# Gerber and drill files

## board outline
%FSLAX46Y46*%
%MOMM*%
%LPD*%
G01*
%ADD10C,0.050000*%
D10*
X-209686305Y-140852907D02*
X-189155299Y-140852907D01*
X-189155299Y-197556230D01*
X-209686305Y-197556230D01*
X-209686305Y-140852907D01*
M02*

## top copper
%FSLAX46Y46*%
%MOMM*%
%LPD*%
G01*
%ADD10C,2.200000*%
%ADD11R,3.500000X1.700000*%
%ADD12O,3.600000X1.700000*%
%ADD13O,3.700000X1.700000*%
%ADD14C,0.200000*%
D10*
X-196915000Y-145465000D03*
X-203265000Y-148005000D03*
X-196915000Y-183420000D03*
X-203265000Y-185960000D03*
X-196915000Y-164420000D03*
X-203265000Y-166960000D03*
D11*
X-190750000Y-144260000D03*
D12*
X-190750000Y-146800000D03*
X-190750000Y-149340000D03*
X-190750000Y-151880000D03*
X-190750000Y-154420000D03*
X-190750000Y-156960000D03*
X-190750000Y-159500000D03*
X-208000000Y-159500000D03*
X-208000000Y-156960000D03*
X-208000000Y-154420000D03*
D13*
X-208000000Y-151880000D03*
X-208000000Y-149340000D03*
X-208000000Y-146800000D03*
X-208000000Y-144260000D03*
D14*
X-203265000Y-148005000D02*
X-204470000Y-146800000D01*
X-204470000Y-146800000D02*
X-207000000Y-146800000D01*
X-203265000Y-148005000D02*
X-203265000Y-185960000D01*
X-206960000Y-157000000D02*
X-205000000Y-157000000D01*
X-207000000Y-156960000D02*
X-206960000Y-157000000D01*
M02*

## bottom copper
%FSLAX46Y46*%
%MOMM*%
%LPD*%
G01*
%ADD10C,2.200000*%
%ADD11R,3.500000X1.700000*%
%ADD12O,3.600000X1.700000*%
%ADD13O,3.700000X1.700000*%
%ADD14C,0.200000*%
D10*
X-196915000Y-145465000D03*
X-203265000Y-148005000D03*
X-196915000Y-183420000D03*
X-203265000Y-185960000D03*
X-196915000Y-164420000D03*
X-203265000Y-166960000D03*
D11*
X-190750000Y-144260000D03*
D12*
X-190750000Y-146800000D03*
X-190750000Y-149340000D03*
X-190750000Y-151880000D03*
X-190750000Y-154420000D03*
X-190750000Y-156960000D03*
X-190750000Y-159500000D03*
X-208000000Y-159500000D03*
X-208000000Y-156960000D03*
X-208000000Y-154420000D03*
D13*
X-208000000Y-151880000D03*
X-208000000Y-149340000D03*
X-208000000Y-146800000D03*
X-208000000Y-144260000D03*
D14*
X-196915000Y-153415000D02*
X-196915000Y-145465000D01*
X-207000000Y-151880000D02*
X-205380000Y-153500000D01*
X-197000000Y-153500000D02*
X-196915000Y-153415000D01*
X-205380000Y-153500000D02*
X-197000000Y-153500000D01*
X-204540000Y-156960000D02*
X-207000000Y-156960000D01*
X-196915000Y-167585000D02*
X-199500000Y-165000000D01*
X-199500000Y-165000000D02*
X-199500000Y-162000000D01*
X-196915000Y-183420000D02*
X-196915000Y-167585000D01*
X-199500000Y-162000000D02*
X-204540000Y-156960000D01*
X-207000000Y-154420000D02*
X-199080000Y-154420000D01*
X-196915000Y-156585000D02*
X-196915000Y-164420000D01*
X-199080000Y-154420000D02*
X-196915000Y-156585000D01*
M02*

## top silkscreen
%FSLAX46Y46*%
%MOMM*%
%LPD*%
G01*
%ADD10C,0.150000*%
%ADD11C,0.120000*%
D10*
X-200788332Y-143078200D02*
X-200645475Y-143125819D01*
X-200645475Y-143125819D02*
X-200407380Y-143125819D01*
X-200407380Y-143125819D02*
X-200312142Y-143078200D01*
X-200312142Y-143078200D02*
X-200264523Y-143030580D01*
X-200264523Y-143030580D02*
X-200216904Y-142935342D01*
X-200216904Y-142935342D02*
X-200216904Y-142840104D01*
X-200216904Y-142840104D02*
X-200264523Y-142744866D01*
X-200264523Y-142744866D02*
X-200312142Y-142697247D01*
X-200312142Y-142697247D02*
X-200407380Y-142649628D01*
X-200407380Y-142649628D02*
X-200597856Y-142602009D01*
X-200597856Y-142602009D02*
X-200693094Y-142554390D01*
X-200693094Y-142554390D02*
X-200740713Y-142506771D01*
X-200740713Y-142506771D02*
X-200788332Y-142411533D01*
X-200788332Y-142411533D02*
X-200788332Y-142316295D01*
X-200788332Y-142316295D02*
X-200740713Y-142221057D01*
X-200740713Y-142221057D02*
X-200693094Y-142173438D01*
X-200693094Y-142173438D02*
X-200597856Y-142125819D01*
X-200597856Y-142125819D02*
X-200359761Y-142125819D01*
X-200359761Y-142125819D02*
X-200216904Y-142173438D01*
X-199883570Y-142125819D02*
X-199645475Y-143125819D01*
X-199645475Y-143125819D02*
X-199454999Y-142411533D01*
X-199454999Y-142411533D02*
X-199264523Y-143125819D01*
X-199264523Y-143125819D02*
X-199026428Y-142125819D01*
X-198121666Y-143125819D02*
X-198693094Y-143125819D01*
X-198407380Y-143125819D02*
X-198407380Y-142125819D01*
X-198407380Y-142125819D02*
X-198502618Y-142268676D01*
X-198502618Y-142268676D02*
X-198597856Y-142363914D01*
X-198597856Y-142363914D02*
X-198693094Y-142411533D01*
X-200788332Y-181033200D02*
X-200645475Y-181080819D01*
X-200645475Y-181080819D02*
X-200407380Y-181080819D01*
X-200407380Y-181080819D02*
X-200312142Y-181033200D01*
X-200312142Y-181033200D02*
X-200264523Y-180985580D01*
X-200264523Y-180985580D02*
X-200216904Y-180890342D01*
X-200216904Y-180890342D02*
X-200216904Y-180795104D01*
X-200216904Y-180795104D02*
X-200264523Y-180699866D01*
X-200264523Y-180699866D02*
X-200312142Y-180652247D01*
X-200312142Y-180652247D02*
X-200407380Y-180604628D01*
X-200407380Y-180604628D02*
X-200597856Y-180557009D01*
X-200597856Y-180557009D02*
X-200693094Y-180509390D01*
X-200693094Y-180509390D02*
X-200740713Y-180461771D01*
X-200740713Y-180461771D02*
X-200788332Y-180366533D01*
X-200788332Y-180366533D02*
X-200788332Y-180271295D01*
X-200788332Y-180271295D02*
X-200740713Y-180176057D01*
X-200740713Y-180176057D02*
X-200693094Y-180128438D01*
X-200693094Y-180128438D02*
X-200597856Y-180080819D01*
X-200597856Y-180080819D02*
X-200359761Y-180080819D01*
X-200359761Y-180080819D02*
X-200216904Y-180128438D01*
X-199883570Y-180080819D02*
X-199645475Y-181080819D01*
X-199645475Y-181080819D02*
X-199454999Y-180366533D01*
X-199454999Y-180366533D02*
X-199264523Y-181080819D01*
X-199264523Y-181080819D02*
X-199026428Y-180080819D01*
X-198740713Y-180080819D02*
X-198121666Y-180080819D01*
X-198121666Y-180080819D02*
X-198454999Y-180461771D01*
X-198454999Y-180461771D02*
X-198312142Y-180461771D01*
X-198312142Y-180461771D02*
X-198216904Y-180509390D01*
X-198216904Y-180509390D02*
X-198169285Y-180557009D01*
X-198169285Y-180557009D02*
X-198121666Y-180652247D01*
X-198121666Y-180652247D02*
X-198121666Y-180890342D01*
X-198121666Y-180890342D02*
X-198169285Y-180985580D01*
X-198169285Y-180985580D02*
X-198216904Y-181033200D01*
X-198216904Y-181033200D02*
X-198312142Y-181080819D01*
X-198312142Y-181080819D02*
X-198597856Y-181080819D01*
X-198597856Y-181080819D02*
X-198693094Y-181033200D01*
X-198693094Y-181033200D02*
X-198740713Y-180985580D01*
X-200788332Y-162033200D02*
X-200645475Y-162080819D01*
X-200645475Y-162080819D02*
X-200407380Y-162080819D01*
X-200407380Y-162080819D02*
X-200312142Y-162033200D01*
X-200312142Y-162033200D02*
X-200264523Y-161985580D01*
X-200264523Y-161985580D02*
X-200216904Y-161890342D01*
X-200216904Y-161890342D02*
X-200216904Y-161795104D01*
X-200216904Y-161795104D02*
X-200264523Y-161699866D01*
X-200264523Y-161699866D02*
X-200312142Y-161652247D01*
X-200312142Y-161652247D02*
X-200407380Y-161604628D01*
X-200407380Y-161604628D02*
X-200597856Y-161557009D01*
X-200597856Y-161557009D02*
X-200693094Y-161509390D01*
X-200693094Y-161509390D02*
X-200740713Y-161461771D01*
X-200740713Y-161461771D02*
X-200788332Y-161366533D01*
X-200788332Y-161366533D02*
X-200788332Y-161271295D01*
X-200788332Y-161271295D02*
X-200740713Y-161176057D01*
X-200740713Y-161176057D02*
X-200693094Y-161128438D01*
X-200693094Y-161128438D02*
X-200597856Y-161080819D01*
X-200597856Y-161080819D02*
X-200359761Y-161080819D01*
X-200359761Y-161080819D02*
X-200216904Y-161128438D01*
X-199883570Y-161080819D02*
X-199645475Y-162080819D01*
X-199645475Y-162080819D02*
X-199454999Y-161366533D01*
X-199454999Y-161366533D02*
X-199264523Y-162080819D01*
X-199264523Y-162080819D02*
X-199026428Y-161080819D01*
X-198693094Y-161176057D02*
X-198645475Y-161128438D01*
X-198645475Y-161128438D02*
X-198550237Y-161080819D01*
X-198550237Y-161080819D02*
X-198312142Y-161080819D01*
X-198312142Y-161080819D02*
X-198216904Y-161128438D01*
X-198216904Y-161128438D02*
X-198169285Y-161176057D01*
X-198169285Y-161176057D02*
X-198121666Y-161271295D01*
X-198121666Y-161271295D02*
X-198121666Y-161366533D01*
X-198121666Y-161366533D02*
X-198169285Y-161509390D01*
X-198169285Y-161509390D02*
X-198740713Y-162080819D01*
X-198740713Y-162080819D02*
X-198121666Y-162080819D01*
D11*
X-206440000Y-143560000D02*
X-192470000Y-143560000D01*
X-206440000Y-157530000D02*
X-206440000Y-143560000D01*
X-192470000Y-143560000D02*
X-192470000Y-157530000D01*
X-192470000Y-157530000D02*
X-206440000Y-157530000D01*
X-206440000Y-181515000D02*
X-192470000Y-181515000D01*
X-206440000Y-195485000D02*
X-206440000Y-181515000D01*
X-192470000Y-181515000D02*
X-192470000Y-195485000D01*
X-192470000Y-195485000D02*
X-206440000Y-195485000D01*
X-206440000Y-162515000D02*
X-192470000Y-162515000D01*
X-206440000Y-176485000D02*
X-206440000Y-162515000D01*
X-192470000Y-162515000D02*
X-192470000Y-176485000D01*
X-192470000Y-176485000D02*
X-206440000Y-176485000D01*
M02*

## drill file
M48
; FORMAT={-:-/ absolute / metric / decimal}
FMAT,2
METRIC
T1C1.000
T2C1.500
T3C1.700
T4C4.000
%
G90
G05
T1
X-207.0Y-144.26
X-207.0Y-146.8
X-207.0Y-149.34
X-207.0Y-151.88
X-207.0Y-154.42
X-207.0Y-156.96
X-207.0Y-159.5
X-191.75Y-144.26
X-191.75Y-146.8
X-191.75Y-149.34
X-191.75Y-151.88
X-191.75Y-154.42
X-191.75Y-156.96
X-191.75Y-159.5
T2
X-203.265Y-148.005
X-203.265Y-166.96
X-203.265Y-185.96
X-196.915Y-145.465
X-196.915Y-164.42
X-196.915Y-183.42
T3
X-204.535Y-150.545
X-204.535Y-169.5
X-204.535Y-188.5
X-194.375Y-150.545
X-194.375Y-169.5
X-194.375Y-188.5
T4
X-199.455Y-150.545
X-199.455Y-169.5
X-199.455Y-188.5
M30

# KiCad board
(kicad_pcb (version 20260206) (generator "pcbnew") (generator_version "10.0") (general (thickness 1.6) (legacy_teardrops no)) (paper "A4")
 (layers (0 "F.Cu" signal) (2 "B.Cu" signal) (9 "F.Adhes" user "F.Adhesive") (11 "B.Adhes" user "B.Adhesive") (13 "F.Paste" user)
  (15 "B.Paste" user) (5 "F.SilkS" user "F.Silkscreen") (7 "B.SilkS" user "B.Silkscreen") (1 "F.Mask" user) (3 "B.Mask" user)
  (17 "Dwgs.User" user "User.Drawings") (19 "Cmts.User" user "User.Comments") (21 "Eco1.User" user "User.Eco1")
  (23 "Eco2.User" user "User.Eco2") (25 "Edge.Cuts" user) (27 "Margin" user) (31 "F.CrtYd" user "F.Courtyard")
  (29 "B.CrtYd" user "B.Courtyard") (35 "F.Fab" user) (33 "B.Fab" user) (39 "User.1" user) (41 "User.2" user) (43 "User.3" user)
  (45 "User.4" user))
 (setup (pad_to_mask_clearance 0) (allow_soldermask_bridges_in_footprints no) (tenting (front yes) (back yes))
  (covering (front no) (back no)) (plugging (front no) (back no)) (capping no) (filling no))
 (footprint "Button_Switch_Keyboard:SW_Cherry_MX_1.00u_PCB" (layer "F.Cu") (at -196.915 145.465)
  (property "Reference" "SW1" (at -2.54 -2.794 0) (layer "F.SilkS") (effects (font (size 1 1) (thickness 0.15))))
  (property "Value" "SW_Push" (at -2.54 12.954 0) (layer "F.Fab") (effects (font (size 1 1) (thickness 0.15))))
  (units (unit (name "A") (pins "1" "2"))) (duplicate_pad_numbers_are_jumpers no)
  (fp_line (start -9.525 -1.905) (end 4.445 -1.905) (stroke (width 0.12) (type solid)) (layer "F.SilkS"))
  (fp_line (start -9.525 12.065) (end -9.525 -1.905) (stroke (width 0.12) (type solid)) (layer "F.SilkS"))
  (fp_line (start 4.445 -1.905) (end 4.445 12.065) (stroke (width 0.12) (type solid)) (layer "F.SilkS"))
  (fp_line (start 4.445 12.065) (end -9.525 12.065) (stroke (width 0.12) (type solid)) (layer "F.SilkS"))
  (pad "" np_thru_hole circle (at -7.62 5.08) (size 1.7 1.7) (drill 1.7) (layers "*.Cu" "*.Mask"))
  (pad "" np_thru_hole circle (at -2.54 5.08) (size 4 4) (drill 4) (layers "*.Cu" "*.Mask"))
  (pad "" np_thru_hole circle (at 2.54 5.08) (size 1.7 1.7) (drill 1.7) (layers "*.Cu" "*.Mask"))
  (pad "1" thru_hole circle (at 0 0) (size 2.2 2.2) (drill 1.5) (layers "*.Cu" "*.Mask") (remove_unused_layers no)
   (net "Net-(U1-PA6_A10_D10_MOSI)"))
  (pad "2" thru_hole circle (at -6.35 2.54) (size 2.2 2.2) (drill 1.5) (layers "*.Cu" "*.Mask") (remove_unused_layers no) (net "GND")))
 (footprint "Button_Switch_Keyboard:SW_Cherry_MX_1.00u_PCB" (layer "F.Cu") (at -196.915 183.42)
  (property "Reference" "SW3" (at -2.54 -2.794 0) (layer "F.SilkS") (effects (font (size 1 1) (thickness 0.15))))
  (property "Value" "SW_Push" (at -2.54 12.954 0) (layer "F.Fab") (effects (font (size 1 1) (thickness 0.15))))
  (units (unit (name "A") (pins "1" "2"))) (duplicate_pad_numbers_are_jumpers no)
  (fp_line (start -9.525 -1.905) (end 4.445 -1.905) (stroke (width 0.12) (type solid)) (layer "F.SilkS"))
  (fp_line (start -9.525 12.065) (end -9.525 -1.905) (stroke (width 0.12) (type solid)) (layer "F.SilkS"))
  (fp_line (start 4.445 -1.905) (end 4.445 12.065) (stroke (width 0.12) (type solid)) (layer "F.SilkS"))
  (fp_line (start 4.445 12.065) (end -9.525 12.065) (stroke (width 0.12) (type solid)) (layer "F.SilkS"))
  (pad "" np_thru_hole circle (at -7.62 5.08) (size 1.7 1.7) (drill 1.7) (layers "*.Cu" "*.Mask"))
  (pad "" np_thru_hole circle (at -2.54 5.08) (size 4 4) (drill 4) (layers "*.Cu" "*.Mask"))
  (pad "" np_thru_hole circle (at 2.54 5.08) (size 1.7 1.7) (drill 1.7) (layers "*.Cu" "*.Mask"))
  (pad "1" thru_hole circle (at 0 0) (size 2.2 2.2) (drill 1.5) (layers "*.Cu" "*.Mask") (remove_unused_layers no)
   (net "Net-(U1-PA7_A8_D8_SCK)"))
  (pad "2" thru_hole circle (at -6.35 2.54) (size 2.2 2.2) (drill 1.5) (layers "*.Cu" "*.Mask") (remove_unused_layers no) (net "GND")))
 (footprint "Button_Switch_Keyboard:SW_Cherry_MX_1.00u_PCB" (layer "F.Cu") (at -196.915 164.42)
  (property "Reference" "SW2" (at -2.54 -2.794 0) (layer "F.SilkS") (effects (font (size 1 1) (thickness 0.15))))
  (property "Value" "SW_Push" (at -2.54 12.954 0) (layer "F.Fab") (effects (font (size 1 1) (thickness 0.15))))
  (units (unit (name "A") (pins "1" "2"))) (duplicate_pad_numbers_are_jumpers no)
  (fp_line (start -9.525 -1.905) (end 4.445 -1.905) (stroke (width 0.12) (type solid)) (layer "F.SilkS"))
  (fp_line (start -9.525 12.065) (end -9.525 -1.905) (stroke (width 0.12) (type solid)) (layer "F.SilkS"))
  (fp_line (start 4.445 -1.905) (end 4.445 12.065) (stroke (width 0.12) (type solid)) (layer "F.SilkS"))
  (fp_line (start 4.445 12.065) (end -9.525 12.065) (stroke (width 0.12) (type solid)) (layer "F.SilkS"))
  (pad "" np_thru_hole circle (at -7.62 5.08) (size 1.7 1.7) (drill 1.7) (layers "*.Cu" "*.Mask"))
  (pad "" np_thru_hole circle (at -2.54 5.08) (size 4 4) (drill 4) (layers "*.Cu" "*.Mask"))
  (pad "" np_thru_hole circle (at 2.54 5.08) (size 1.7 1.7) (drill 1.7) (layers "*.Cu" "*.Mask"))
  (pad "1" thru_hole circle (at 0 0) (size 2.2 2.2) (drill 1.5) (layers "*.Cu" "*.Mask") (remove_unused_layers no)
   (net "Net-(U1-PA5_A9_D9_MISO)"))
  (pad "2" thru_hole circle (at -6.35 2.54) (size 2.2 2.2) (drill 1.5) (layers "*.Cu" "*.Mask") (remove_unused_layers no) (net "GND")))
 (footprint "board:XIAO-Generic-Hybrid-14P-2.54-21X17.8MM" (layer "B.Cu") (at -199.375 151.88 180)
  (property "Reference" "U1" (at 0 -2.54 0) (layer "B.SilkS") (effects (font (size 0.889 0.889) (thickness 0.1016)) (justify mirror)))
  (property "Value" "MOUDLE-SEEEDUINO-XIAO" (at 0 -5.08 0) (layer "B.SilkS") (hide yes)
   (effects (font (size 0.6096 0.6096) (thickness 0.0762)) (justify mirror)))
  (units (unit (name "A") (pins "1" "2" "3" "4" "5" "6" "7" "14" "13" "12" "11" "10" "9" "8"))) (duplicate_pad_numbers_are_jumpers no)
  (pad "1" thru_hole rect (at -7.625 7.62 180) (size 3.5 1.7) (drill 1 (offset -1 0)) (layers "*.Cu" "*.Mask") (remove_unused_layers no)
   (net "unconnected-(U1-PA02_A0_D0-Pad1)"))
  (pad "2" thru_hole oval (at -7.625 5.08 180) (size 3.6 1.7) (drill 1 (offset -1 0)) (layers "*.Cu" "*.Mask") (remove_unused_layers no)
   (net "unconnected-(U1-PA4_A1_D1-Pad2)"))
  (pad "3" thru_hole oval (at -7.625 2.54 180) (size 3.6 1.7) (drill 1 (offset -1 0)) (layers "*.Cu" "*.Mask") (remove_unused_layers no)
   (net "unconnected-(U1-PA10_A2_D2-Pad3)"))
  (pad "4" thru_hole oval (at -7.625 0 180) (size 3.6 1.7) (drill 1 (offset -1 0)) (layers "*.Cu" "*.Mask") (remove_unused_layers no)
   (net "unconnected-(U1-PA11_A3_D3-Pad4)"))
  (pad "5" thru_hole oval (at -7.625 -2.54 180) (size 3.6 1.7) (drill 1 (offset -1 0)) (layers "*.Cu" "*.Mask") (remove_unused_layers no)
   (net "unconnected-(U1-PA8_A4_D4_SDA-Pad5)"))
  (pad "6" thru_hole oval (at -7.625 -5.08) (size 3.6 1.7) (drill 1 (offset 1 0)) (layers "*.Cu" "*.Mask") (remove_unused_layers no)
   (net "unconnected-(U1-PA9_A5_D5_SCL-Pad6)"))
  (pad "7" thru_hole oval (at -7.625 -7.62 180) (size 3.6 1.7) (drill 1 (offset -1 0)) (layers "*.Cu" "*.Mask") (remove_unused_layers no)
   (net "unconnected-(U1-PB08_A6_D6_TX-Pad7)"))
  (pad "8" thru_hole oval (at 7.625 -7.62 180) (size 3.6 1.7) (drill 1 (offset 1 0)) (layers "*.Cu" "*.Mask") (remove_unused_layers no)
   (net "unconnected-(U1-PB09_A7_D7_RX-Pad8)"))
  (pad "9" thru_hole oval (at 7.625 -5.08 180) (size 3.6 1.7) (drill 1 (offset 1 0)) (layers "*.Cu" "*.Mask") (remove_unused_layers no)
   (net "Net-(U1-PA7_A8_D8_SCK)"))
  (pad "10" thru_hole oval (at 7.625 -2.54 180) (size 3.6 1.7) (drill 1 (offset 1 0)) (layers "*.Cu" "*.Mask") (remove_unused_layers no)
   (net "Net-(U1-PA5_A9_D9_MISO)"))
  (pad "11" thru_hole oval (at 7.625 0 180) (size 3.7 1.7) (drill 1 (offset 1 0)) (layers "*.Cu" "*.Mask") (remove_unused_layers no)
   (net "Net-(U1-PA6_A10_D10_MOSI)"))
  (pad "12" thru_hole oval (at 7.625 2.54 180) (size 3.7 1.7) (drill 1 (offset 1 0)) (layers "*.Cu" "*.Mask") (remove_unused_layers no)
   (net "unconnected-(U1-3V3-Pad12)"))
  (pad "13" thru_hole oval (at 7.625 5.08 180) (size 3.7 1.7) (drill 1 (offset 1 0)) (layers "*.Cu" "*.Mask") (remove_unused_layers no)
   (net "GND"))
  (pad "14" thru_hole oval (at 7.625 7.62 180) (size 3.7 1.7) (drill 1 (offset 1 0)) (layers "*.Cu" "*.Mask") (remove_unused_layers no)
   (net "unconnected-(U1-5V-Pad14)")))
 (gr_rect (start -209.686305 140.852907) (end -189.155299 197.55623) (stroke (width 0.05) (type default)) (fill no) (layer "Edge.Cuts"))
 (segment (start -196.915 153.415) (end -196.915 145.465) (width 0.2) (layer "B.Cu") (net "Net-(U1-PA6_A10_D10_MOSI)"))
 (segment (start -207 151.88) (end -205.38 153.5) (width 0.2) (layer "B.Cu") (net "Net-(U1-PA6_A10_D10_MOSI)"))
 (segment (start -197 153.5) (end -196.915 153.415) (width 0.2) (layer "B.Cu") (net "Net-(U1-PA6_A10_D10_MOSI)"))
 (segment (start -205.38 153.5) (end -197 153.5) (width 0.2) (layer "B.Cu") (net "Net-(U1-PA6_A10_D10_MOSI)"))
 (segment (start -203.265 148.005) (end -204.47 146.8) (width 0.2) (layer "F.Cu") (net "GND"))
 (segment (start -204.47 146.8) (end -207 146.8) (width 0.2) (layer "F.Cu") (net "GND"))
 (segment (start -203.265 148.005) (end -203.265 185.96) (width 0.2) (layer "F.Cu") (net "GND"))
 (segment (start -206.96 157) (end -205 157) (width 0.2) (layer "F.Cu") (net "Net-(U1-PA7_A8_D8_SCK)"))
 (segment (start -207 156.96) (end -206.96 157) (width 0.2) (layer "F.Cu") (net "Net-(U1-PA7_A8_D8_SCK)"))
 (segment (start -204.54 156.96) (end -207 156.96) (width 0.2) (layer "B.Cu") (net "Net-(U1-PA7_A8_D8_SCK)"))
 (segment (start -196.915 167.585) (end -199.5 165) (width 0.2) (layer "B.Cu") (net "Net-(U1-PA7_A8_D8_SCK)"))
 (segment (start -199.5 165) (end -199.5 162) (width 0.2) (layer "B.Cu") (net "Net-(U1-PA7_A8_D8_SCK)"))
 (segment (start -196.915 183.42) (end -196.915 167.585) (width 0.2) (layer "B.Cu") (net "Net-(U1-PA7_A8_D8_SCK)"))
 (segment (start -199.5 162) (end -204.54 156.96) (width 0.2) (layer "B.Cu") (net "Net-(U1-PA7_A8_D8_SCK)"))
 (segment (start -207 154.42) (end -199.08 154.42) (width 0.2) (layer "B.Cu") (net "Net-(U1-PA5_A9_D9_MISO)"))
 (segment (start -196.915 156.585) (end -196.915 164.42) (width 0.2) (layer "B.Cu") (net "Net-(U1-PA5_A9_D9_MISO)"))
 (segment (start -199.08 154.42) (end -196.915 156.585) (width 0.2) (layer "B.Cu") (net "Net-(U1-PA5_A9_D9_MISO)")))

